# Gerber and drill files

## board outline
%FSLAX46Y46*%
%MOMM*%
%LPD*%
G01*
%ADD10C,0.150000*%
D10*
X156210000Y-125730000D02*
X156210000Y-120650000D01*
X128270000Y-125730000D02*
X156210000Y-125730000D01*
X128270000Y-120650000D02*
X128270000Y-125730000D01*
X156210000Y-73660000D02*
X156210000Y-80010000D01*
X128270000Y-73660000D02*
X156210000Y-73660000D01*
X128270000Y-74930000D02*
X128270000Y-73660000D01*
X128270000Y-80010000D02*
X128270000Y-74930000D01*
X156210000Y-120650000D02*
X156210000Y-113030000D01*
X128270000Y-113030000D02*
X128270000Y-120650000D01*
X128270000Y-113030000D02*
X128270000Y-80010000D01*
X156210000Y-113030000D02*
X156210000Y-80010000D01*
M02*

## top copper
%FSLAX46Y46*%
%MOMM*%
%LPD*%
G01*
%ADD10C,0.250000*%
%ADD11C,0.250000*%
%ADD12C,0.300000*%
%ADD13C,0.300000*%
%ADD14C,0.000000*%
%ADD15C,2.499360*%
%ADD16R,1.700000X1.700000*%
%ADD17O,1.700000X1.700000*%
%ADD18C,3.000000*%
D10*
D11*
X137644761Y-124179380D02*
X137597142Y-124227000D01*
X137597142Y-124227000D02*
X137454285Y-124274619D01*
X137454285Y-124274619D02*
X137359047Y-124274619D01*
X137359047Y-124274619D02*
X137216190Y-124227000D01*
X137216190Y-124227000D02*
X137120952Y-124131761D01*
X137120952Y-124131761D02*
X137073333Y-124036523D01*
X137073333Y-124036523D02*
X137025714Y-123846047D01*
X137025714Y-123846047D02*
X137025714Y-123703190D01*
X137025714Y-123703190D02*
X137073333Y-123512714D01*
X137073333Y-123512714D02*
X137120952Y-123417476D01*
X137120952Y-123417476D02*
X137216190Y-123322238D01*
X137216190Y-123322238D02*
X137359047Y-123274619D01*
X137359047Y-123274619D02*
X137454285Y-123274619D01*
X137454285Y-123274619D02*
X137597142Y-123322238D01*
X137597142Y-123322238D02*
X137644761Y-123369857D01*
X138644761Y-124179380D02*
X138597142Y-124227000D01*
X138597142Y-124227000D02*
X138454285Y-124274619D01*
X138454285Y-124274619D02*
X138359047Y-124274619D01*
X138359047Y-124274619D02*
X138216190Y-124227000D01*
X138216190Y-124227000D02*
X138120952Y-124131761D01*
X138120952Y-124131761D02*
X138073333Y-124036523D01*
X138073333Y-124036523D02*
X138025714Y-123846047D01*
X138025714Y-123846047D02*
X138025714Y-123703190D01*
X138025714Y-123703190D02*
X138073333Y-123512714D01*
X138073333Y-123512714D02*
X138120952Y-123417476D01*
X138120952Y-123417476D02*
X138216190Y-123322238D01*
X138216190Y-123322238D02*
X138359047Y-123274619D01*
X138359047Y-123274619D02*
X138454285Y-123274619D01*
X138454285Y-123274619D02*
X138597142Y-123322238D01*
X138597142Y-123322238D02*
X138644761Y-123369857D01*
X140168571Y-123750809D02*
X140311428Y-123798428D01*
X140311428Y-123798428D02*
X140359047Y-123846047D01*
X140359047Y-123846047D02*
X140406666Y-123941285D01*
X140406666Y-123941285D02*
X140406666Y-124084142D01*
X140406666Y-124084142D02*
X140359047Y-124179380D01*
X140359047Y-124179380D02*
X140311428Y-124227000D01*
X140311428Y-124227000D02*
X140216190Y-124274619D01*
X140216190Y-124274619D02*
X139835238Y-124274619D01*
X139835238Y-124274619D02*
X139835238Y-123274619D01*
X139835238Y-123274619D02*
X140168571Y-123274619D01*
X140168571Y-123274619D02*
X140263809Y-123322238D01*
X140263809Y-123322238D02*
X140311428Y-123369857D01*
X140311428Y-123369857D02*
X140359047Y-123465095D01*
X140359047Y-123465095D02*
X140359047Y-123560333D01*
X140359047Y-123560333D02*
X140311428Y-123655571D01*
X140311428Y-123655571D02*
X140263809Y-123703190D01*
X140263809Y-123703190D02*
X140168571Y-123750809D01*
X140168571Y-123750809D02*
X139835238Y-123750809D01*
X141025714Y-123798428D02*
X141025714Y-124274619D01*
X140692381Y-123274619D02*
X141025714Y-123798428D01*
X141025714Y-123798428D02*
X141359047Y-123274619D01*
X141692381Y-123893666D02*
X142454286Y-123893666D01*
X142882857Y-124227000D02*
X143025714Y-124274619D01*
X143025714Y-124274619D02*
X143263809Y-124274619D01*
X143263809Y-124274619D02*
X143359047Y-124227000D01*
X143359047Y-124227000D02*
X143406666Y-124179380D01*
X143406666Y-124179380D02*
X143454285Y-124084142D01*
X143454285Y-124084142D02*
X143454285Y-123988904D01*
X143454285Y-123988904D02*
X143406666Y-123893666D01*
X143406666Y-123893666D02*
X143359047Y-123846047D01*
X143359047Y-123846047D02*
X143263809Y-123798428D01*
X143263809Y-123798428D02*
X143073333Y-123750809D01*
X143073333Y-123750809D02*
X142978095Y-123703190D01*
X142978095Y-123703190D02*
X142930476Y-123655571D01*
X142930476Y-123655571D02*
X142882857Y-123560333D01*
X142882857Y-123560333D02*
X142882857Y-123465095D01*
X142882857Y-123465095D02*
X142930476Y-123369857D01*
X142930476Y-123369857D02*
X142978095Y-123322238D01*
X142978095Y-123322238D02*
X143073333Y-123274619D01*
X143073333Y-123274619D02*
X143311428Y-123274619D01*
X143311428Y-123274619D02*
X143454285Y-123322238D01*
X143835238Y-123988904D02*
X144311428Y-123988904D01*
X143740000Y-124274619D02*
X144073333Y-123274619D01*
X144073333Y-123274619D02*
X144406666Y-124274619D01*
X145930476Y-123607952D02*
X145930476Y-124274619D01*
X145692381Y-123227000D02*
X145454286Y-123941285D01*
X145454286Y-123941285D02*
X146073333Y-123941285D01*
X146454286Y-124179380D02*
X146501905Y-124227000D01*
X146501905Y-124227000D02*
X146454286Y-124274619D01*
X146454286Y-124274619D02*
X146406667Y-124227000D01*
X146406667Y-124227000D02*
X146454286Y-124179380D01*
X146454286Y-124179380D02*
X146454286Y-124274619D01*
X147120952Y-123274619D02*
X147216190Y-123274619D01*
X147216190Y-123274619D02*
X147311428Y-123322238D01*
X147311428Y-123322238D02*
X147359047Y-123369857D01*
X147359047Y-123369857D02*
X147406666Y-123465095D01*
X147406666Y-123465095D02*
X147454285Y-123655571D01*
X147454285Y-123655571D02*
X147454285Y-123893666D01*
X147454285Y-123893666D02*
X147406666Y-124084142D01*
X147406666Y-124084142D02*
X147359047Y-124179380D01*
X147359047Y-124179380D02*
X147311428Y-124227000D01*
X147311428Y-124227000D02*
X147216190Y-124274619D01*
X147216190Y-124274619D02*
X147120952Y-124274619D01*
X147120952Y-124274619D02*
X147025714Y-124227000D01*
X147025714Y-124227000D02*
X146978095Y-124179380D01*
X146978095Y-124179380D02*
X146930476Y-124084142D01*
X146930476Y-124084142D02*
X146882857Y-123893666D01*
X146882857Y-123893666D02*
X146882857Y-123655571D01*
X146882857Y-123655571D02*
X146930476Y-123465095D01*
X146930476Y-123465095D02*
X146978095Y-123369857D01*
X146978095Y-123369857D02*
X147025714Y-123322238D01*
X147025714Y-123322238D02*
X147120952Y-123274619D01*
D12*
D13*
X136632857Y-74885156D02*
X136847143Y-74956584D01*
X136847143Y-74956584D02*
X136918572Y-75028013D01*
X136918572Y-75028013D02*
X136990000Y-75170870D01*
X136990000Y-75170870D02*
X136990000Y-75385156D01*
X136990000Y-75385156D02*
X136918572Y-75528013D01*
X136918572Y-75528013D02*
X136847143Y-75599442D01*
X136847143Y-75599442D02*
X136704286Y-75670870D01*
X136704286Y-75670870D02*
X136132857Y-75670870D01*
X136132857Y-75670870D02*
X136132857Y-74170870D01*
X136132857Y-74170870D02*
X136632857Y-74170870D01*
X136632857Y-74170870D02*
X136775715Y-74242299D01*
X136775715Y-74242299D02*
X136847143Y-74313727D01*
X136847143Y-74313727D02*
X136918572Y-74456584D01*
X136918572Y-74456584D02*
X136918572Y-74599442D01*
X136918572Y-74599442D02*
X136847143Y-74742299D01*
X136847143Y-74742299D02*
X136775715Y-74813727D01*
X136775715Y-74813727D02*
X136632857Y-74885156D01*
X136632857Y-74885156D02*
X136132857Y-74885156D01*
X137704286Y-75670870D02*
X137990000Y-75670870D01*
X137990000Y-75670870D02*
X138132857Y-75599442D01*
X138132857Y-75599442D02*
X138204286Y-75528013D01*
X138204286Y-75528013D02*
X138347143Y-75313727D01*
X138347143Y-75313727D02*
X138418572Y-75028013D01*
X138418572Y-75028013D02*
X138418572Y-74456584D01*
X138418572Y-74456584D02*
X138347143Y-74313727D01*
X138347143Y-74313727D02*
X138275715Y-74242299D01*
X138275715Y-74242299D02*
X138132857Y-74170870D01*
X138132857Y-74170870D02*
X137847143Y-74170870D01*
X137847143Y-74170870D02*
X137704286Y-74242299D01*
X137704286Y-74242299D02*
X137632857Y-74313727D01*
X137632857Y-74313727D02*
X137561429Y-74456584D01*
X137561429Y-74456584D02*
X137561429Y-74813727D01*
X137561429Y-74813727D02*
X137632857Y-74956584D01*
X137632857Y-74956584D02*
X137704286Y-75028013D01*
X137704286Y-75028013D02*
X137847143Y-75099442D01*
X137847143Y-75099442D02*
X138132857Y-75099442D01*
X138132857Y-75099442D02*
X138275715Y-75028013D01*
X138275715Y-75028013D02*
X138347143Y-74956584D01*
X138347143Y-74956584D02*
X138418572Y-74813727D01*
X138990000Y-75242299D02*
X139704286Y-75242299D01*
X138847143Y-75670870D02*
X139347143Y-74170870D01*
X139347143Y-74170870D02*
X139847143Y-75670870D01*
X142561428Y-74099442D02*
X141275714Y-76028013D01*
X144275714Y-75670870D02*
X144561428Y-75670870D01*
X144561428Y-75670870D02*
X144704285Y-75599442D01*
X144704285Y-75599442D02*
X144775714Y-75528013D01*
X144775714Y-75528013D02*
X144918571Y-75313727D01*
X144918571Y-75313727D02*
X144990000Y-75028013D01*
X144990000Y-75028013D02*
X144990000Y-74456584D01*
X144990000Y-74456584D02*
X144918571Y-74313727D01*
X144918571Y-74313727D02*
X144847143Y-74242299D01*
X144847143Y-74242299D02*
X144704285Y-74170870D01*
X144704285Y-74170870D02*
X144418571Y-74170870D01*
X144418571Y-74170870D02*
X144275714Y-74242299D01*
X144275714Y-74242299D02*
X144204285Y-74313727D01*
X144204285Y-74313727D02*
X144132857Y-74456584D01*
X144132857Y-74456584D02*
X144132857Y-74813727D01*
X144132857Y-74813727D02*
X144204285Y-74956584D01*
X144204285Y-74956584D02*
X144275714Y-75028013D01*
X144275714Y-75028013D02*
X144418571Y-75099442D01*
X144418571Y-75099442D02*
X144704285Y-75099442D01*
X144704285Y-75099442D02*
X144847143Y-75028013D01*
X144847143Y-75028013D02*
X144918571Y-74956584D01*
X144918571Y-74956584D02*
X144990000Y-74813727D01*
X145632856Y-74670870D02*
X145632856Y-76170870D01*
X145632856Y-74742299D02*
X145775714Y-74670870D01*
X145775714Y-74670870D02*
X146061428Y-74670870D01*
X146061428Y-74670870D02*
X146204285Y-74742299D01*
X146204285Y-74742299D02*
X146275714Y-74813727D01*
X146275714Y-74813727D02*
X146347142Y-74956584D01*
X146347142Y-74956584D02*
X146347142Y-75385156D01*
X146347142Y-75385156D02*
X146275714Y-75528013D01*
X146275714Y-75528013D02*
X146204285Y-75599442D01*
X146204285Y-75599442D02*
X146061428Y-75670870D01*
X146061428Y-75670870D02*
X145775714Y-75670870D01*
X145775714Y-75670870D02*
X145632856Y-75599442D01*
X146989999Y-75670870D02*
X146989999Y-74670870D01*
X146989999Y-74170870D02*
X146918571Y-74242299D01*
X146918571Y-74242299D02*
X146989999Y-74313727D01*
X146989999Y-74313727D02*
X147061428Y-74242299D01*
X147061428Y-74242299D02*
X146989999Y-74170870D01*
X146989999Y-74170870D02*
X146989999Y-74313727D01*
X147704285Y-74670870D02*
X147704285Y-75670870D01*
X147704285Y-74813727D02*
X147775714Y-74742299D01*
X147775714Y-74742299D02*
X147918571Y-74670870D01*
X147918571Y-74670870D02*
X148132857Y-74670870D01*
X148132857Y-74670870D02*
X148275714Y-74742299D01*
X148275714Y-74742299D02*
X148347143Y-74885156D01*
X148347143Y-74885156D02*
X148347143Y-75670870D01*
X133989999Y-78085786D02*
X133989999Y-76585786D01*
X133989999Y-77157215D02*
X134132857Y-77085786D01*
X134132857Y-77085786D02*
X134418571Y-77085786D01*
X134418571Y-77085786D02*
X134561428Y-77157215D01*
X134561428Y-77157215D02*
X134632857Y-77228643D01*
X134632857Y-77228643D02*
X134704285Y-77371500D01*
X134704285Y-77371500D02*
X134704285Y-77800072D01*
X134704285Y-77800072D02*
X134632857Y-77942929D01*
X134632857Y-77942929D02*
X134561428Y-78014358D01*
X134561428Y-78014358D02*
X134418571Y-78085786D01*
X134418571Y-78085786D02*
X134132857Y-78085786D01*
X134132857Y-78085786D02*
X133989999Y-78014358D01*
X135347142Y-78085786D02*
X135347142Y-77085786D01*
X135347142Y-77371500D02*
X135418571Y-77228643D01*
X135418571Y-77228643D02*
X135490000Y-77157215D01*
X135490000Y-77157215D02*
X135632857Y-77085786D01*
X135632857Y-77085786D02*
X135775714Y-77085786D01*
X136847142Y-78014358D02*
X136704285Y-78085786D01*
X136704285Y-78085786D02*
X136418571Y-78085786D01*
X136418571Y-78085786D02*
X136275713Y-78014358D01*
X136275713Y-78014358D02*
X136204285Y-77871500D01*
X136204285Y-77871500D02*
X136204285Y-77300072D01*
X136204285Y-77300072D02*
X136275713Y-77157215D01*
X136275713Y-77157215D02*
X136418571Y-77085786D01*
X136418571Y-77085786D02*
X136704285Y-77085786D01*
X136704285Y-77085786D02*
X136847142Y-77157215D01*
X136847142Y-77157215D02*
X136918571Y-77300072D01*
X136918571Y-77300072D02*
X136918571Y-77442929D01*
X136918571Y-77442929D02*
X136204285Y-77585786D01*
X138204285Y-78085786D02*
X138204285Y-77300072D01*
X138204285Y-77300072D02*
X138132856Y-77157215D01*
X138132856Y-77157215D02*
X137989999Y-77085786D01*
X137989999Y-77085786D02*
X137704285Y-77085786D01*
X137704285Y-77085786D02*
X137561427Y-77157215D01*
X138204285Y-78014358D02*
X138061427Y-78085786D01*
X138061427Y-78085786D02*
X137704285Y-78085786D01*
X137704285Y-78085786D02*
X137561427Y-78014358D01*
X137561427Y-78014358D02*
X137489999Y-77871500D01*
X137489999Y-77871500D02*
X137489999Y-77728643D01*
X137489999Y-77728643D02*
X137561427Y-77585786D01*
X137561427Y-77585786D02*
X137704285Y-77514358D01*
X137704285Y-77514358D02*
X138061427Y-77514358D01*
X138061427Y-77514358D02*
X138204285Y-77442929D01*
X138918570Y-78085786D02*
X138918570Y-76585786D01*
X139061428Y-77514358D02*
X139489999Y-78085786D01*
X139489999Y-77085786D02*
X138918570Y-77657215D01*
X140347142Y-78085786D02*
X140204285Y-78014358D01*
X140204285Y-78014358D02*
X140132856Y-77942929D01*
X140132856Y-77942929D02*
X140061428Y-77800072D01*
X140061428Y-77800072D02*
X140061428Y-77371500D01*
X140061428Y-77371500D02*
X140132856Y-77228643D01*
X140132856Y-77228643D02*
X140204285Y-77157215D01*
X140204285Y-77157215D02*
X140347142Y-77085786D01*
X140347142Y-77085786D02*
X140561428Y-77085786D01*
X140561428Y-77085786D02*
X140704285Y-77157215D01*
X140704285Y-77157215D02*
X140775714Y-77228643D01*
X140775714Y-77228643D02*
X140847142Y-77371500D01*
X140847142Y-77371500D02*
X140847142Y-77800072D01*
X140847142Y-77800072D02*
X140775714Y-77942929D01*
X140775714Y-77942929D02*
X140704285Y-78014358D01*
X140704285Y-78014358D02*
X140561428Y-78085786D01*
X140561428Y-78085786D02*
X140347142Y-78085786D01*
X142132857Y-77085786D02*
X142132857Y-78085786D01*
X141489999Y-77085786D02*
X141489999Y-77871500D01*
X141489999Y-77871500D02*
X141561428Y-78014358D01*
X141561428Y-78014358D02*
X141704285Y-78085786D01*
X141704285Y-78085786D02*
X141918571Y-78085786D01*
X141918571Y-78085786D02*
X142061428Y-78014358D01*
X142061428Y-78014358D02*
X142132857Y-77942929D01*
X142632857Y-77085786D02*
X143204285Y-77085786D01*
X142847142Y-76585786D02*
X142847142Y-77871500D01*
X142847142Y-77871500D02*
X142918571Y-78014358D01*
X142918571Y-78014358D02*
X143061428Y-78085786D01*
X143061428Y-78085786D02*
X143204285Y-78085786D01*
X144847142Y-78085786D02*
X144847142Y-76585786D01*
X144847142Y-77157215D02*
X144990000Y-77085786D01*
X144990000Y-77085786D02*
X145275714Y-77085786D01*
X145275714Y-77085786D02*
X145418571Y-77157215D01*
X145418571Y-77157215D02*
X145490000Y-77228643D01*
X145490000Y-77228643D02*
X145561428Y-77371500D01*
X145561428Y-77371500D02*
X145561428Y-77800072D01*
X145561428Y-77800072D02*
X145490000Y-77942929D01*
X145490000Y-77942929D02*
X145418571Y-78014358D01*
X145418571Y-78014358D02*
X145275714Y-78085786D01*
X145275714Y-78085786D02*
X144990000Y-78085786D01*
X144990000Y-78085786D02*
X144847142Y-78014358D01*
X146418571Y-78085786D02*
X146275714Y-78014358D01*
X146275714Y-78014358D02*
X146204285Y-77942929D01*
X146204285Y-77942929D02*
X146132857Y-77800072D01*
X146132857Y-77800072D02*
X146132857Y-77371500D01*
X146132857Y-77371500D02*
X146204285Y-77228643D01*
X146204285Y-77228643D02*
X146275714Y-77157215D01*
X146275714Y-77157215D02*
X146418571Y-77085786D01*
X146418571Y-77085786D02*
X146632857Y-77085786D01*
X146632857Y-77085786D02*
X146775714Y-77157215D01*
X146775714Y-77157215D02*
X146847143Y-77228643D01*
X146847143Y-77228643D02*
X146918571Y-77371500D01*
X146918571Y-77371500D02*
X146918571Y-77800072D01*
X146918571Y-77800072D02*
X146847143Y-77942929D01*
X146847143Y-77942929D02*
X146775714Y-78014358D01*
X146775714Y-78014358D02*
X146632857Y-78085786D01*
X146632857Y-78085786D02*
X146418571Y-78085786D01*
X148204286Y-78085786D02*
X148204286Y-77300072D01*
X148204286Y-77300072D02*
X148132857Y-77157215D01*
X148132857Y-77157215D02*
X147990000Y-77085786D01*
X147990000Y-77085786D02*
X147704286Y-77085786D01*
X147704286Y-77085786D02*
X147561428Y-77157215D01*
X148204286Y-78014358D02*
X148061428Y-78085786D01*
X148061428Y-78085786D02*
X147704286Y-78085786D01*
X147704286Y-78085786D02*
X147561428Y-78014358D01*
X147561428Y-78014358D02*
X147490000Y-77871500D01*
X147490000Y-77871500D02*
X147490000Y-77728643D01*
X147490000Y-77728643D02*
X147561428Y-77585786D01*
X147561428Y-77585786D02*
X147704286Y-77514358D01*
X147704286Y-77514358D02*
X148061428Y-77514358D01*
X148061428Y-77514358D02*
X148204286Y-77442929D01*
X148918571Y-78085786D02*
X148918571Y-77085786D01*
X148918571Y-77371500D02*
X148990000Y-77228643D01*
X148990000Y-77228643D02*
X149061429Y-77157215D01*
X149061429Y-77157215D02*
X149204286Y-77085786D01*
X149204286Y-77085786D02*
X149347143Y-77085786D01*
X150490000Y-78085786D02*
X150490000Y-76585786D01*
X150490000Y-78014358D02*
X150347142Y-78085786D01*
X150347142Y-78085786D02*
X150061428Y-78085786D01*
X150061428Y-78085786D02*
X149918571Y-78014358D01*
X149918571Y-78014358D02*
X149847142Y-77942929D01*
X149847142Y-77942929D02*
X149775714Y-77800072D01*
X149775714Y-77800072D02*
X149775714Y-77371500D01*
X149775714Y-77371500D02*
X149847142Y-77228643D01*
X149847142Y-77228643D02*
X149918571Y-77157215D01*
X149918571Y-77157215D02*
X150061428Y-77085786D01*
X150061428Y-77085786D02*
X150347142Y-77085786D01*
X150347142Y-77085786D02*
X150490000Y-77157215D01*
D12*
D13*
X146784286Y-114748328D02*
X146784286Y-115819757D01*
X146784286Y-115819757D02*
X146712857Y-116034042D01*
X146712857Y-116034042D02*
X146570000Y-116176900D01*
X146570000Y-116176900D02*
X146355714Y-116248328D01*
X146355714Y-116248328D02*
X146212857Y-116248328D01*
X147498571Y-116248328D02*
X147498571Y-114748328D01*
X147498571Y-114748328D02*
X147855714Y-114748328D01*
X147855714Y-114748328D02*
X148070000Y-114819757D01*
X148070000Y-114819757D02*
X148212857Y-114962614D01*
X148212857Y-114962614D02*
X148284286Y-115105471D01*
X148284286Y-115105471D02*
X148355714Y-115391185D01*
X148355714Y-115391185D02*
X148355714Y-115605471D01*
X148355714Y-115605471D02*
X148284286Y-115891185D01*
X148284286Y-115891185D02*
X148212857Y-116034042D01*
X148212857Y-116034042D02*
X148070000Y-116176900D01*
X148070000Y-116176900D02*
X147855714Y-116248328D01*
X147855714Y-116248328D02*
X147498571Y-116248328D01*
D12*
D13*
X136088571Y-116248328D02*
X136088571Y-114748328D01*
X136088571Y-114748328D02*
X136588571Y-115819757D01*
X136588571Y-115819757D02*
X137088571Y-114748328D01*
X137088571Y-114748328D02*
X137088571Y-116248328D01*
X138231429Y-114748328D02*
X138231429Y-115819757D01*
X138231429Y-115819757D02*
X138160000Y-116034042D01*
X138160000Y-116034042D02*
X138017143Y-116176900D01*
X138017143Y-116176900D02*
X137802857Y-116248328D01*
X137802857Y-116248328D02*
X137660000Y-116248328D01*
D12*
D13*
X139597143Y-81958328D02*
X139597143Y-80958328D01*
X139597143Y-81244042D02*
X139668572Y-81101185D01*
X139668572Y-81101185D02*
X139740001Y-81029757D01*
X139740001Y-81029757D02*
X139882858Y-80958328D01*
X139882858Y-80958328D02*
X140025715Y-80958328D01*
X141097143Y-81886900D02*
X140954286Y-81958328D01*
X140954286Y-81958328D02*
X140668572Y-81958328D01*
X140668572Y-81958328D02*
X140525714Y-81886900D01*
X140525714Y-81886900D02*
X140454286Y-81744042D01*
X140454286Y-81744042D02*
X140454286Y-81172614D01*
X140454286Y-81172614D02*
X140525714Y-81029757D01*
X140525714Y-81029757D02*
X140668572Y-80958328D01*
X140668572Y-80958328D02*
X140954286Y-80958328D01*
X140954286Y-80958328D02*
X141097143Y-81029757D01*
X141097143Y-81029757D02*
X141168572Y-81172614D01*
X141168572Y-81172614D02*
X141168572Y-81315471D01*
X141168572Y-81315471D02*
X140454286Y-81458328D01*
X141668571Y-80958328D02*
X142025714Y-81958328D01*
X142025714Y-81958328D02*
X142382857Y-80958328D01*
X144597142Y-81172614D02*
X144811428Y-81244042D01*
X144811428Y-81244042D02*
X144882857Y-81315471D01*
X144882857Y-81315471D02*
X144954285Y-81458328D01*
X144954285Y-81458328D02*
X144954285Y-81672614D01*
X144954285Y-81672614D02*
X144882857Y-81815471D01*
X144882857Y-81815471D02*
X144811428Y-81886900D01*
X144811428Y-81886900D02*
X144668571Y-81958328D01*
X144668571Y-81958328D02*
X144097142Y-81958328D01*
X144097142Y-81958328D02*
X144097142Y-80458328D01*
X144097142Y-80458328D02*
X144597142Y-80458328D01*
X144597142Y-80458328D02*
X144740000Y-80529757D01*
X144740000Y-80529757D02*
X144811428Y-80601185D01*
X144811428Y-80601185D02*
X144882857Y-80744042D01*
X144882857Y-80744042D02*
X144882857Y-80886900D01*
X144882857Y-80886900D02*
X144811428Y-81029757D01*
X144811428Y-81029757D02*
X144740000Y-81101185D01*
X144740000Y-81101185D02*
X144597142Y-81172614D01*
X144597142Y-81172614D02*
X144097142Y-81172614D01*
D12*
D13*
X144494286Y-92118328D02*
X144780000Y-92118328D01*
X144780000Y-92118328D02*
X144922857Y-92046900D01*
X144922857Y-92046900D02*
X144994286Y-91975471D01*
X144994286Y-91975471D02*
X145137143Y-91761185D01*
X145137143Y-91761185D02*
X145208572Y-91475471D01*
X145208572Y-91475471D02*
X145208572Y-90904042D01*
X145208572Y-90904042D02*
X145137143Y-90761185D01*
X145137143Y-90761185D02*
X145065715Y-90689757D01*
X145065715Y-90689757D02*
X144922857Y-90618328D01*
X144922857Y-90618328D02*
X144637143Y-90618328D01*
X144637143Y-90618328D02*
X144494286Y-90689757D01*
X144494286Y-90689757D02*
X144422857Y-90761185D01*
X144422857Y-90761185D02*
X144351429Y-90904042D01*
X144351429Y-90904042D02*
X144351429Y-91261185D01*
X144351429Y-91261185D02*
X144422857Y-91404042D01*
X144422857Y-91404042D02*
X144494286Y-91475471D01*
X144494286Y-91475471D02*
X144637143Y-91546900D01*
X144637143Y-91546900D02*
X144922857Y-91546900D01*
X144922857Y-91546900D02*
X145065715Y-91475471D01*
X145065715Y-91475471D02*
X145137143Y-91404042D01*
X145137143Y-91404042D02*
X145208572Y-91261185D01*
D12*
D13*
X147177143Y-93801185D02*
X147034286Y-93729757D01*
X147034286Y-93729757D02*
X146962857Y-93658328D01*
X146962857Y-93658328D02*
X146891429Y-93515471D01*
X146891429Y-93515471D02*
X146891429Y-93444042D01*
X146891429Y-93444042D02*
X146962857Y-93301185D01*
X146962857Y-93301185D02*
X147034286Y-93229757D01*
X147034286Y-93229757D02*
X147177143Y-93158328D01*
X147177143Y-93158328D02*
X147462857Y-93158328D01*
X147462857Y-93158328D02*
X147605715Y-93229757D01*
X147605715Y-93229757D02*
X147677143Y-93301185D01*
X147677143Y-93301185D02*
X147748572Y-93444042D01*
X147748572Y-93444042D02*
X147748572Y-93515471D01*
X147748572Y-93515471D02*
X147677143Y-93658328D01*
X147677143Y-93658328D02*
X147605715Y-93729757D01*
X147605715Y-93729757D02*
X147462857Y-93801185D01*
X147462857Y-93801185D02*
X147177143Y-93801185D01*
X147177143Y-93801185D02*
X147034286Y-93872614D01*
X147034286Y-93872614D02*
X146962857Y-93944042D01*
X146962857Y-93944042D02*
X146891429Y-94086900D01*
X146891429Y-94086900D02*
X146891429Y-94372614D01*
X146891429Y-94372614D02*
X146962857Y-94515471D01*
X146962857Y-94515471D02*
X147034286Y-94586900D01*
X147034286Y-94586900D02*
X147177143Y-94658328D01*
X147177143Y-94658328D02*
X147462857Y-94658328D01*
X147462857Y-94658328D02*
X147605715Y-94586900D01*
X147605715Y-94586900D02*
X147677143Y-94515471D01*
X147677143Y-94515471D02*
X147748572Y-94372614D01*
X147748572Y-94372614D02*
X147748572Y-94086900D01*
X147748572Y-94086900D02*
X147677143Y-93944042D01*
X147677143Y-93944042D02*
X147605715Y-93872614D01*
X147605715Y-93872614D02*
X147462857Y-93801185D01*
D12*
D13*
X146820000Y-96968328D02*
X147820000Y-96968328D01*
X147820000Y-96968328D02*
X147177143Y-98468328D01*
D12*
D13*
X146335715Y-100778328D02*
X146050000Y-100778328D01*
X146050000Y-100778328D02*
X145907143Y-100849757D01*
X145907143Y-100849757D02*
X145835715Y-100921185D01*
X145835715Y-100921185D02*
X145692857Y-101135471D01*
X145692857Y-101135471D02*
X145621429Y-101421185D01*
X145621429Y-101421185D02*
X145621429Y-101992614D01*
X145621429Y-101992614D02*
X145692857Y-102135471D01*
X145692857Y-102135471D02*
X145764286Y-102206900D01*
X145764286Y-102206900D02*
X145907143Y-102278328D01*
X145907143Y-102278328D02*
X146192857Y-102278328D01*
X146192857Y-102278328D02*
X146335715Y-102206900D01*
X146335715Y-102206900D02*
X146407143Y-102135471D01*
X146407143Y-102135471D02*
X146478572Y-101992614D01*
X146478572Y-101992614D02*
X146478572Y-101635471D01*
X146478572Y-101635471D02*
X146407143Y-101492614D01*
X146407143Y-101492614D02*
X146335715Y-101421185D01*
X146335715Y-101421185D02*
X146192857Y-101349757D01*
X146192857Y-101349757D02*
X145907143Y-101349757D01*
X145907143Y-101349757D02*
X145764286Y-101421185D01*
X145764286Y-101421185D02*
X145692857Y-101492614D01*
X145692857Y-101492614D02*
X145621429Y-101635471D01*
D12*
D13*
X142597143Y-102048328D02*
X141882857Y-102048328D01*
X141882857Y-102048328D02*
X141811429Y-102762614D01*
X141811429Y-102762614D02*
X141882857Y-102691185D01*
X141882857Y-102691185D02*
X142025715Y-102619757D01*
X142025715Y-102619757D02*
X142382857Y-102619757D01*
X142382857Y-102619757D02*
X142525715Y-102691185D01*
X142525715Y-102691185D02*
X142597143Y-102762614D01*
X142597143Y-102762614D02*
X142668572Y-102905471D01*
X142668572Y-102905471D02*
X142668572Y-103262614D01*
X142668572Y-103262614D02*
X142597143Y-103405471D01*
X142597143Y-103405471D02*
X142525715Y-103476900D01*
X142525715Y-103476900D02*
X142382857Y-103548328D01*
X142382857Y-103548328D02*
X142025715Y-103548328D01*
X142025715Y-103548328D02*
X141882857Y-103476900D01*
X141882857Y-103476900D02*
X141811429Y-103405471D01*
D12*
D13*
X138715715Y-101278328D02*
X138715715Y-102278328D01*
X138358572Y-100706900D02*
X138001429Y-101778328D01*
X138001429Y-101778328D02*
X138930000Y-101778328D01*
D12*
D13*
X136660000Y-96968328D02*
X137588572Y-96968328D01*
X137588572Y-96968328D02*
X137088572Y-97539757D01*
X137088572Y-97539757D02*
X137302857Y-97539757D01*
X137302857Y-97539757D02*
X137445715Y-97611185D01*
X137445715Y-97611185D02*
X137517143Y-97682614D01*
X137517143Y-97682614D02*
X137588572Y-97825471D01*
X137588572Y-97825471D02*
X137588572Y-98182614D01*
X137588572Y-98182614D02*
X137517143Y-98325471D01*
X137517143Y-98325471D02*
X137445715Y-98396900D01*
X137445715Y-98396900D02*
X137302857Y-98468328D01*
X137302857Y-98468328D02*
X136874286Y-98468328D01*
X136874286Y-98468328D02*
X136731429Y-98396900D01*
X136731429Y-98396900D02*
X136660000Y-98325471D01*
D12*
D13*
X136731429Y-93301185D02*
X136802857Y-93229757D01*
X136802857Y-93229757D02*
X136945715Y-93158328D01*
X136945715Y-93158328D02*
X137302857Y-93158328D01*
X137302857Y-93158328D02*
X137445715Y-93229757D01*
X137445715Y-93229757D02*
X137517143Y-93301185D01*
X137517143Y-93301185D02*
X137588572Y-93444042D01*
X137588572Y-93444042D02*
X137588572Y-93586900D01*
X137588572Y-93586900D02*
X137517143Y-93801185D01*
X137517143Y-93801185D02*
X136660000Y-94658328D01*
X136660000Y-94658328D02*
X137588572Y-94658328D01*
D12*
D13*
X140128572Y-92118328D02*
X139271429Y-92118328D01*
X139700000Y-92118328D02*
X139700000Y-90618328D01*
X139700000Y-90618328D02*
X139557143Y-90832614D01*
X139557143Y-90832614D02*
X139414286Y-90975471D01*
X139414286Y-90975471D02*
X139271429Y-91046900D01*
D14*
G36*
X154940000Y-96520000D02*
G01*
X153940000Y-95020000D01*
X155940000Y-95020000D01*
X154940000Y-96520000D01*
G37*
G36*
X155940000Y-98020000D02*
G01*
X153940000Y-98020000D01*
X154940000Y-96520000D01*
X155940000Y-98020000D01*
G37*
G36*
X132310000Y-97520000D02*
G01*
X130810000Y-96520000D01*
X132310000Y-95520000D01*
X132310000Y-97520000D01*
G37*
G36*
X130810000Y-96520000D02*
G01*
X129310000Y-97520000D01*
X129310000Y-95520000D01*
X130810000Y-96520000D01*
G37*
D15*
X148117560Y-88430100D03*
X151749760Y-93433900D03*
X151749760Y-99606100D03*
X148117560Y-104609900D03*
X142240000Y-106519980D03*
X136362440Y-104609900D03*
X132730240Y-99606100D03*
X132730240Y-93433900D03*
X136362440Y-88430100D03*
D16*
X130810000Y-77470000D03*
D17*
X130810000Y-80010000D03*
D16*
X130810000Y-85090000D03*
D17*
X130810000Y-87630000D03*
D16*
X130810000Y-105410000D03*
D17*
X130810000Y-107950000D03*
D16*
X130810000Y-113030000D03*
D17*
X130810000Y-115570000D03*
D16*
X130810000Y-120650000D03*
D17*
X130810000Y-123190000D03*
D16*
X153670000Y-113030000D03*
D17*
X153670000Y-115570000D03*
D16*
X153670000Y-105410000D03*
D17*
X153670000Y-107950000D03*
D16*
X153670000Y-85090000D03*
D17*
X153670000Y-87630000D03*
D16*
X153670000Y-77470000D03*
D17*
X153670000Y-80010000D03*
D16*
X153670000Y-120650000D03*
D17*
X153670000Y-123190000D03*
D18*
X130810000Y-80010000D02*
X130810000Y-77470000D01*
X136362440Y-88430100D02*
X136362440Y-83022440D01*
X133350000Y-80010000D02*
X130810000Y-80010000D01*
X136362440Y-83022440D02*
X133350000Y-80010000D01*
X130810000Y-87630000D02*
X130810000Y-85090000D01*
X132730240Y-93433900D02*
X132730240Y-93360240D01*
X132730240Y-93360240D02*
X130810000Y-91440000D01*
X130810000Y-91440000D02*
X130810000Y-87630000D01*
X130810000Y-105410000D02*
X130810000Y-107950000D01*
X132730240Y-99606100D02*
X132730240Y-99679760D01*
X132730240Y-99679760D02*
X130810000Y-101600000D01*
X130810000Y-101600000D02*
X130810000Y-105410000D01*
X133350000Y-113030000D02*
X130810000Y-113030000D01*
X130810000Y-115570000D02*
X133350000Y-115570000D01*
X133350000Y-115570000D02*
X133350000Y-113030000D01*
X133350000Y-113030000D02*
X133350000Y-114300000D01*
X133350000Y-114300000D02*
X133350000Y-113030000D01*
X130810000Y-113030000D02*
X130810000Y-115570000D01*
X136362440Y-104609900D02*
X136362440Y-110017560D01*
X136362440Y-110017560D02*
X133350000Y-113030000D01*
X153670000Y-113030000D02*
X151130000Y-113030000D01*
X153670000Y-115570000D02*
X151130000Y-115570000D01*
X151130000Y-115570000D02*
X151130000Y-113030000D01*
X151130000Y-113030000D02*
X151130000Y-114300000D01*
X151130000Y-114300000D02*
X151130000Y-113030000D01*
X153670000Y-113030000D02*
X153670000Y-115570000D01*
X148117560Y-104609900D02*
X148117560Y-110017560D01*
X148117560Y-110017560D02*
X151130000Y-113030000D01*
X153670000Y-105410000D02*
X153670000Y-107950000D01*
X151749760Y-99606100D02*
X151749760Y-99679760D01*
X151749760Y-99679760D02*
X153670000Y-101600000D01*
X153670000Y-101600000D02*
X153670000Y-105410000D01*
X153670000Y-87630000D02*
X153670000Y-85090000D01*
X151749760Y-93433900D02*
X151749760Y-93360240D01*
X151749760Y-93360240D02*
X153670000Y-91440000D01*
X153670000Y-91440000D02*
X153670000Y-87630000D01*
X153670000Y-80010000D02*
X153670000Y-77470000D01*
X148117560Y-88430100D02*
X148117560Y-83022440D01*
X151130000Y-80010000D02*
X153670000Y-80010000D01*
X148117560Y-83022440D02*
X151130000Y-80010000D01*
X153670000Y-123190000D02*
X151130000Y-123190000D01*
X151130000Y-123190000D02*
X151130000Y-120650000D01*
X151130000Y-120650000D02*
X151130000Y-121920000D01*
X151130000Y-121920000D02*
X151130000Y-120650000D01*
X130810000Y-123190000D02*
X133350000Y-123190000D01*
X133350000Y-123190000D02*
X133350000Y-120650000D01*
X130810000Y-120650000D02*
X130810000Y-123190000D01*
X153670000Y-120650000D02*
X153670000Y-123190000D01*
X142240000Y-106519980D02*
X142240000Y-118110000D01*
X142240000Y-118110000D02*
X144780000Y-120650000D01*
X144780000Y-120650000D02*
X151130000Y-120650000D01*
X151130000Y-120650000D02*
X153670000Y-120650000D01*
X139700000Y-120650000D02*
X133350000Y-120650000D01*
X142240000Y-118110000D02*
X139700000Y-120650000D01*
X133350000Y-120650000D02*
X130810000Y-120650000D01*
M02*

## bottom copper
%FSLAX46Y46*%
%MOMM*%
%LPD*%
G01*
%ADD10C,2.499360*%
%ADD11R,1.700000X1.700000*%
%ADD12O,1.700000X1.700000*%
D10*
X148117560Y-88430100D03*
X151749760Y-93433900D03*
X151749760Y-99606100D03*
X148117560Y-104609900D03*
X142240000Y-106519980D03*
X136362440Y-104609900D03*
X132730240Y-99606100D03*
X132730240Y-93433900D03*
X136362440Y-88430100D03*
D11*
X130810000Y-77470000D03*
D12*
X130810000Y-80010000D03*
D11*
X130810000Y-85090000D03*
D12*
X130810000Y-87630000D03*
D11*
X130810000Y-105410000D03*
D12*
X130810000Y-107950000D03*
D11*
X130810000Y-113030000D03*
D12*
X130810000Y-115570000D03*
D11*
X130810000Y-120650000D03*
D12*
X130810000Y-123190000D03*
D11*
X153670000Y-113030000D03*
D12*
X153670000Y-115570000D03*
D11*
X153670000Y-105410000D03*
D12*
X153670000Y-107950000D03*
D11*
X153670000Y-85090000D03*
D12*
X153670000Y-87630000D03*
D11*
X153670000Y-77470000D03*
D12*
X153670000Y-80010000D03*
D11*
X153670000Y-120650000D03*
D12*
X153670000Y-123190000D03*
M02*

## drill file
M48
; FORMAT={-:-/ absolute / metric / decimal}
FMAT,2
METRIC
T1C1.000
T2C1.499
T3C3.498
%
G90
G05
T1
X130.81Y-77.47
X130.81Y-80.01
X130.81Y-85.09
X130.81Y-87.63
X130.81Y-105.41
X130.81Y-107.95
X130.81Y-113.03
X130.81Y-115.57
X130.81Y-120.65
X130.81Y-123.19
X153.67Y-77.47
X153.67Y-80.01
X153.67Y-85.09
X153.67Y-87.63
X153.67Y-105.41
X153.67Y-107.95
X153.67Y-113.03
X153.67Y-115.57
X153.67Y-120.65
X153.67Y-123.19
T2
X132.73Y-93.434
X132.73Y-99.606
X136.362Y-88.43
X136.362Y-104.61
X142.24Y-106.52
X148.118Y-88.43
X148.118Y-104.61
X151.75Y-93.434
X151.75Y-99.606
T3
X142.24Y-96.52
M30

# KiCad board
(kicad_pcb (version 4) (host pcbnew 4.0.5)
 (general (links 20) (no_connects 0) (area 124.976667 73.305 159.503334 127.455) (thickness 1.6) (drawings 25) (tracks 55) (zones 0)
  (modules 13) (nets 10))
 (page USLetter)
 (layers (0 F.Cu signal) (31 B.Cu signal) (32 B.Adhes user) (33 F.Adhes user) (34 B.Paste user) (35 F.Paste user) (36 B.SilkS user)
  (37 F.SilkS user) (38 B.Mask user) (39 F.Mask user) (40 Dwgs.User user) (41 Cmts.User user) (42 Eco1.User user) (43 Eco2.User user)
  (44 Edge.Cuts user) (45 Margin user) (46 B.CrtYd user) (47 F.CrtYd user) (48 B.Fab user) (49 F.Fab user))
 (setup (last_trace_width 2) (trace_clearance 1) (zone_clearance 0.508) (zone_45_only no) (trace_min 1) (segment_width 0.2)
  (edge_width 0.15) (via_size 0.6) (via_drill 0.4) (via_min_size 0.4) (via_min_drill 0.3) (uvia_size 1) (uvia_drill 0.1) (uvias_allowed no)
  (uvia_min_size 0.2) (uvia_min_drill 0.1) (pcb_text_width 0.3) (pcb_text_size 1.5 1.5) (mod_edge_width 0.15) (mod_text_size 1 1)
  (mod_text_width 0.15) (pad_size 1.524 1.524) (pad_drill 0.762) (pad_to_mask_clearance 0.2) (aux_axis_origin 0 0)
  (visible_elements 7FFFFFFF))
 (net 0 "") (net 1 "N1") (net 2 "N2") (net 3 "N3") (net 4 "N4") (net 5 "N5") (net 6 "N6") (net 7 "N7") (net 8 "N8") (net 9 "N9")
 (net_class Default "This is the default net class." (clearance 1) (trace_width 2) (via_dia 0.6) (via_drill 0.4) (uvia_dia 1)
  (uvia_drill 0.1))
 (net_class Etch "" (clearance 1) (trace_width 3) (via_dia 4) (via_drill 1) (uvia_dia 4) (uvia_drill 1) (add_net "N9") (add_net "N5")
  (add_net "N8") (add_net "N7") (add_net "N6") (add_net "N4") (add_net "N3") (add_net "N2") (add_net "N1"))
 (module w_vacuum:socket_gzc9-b (layer F.Cu) (at 142.24 96.52 180)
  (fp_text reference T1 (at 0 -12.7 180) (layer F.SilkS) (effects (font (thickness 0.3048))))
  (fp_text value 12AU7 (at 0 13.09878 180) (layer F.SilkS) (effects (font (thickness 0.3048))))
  (pad 9 thru_hole circle (at -5.87756 8.0899 180) (size 2.49936 2.49936) (drill 1.4986) (layers *.Cu *.Mask F.SilkS) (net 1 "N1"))
  (pad 8 thru_hole circle (at -9.50976 3.0861 180) (size 2.49936 2.49936) (drill 1.4986) (layers *.Cu *.Mask F.SilkS) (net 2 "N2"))
  (pad 7 thru_hole circle (at -9.50976 -3.0861 180) (size 2.49936 2.49936) (drill 1.4986) (layers *.Cu *.Mask F.SilkS) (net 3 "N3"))
  (pad 6 thru_hole circle (at -5.87756 -8.0899 180) (size 2.49936 2.49936) (drill 1.4986) (layers *.Cu *.Mask F.SilkS) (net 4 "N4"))
  (pad 5 thru_hole circle (at 0 -9.99998 180) (size 2.49936 2.49936) (drill 1.4986) (layers *.Cu *.Mask F.SilkS) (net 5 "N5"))
  (pad 4 thru_hole circle (at 5.87756 -8.0899 180) (size 2.49936 2.49936) (drill 1.4986) (layers *.Cu *.Mask F.SilkS) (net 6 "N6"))
  (pad 3 thru_hole circle (at 9.50976 -3.0861 180) (size 2.49936 2.49936) (drill 1.4986) (layers *.Cu *.Mask F.SilkS) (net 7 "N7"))
  (pad 2 thru_hole circle (at 9.50976 3.0861 180) (size 2.49936 2.49936) (drill 1.4986) (layers *.Cu *.Mask F.SilkS) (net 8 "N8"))
  (pad 1 thru_hole circle (at 5.87756 8.0899 180) (size 2.49936 2.49936) (drill 1.4986) (layers *.Cu *.Mask F.SilkS) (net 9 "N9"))
  (pad "" np_thru_hole circle (at 0 0 180) (size 3.49758 3.49758) (drill 3.49758) (layers *.Cu *.Mask F.SilkS)))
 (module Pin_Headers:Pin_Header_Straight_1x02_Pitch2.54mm (layer F.Cu) (at 130.81 77.47)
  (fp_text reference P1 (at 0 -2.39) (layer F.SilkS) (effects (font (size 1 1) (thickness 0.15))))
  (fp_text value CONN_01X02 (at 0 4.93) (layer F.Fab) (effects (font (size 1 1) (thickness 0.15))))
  (pad 1 thru_hole rect (at 0 0) (size 1.7 1.7) (drill 1) (layers *.Cu *.Mask) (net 9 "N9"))
  (pad 2 thru_hole oval (at 0 2.54) (size 1.7 1.7) (drill 1) (layers *.Cu *.Mask) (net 9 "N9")))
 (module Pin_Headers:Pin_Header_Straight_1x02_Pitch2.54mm (layer F.Cu) (at 130.81 85.09)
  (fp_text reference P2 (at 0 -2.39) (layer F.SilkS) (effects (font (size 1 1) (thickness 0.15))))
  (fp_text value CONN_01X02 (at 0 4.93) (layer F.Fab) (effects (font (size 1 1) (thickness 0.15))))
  (pad 1 thru_hole rect (at 0 0) (size 1.7 1.7) (drill 1) (layers *.Cu *.Mask) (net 8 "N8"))
  (pad 2 thru_hole oval (at 0 2.54) (size 1.7 1.7) (drill 1) (layers *.Cu *.Mask) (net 8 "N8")))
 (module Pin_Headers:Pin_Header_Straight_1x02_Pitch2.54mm (layer F.Cu) (at 130.81 105.41)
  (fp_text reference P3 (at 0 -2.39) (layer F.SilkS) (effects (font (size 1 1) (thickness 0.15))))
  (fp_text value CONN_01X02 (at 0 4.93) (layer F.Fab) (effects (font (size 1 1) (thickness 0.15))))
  (pad 1 thru_hole rect (at 0 0) (size 1.7 1.7) (drill 1) (layers *.Cu *.Mask) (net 7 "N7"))
  (pad 2 thru_hole oval (at 0 2.54) (size 1.7 1.7) (drill 1) (layers *.Cu *.Mask) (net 7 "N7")))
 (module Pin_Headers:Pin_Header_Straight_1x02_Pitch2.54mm (layer F.Cu) (at 130.81 113.03)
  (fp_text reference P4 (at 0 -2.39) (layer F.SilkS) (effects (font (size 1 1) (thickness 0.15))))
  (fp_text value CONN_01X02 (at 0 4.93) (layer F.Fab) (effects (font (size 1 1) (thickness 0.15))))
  (pad 1 thru_hole rect (at 0 0) (size 1.7 1.7) (drill 1) (layers *.Cu *.Mask) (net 6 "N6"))
  (pad 2 thru_hole oval (at 0 2.54) (size 1.7 1.7) (drill 1) (layers *.Cu *.Mask) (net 6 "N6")))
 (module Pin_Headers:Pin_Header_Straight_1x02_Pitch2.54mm (layer F.Cu) (at 130.81 120.65)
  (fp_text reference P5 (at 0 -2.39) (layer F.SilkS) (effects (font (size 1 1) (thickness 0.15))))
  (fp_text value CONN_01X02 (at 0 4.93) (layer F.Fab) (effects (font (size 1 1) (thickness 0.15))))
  (pad 1 thru_hole rect (at 0 0) (size 1.7 1.7) (drill 1) (layers *.Cu *.Mask) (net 5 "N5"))
  (pad 2 thru_hole oval (at 0 2.54) (size 1.7 1.7) (drill 1) (layers *.Cu *.Mask) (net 5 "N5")))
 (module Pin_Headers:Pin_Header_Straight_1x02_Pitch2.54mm (layer F.Cu) (at 153.67 113.03)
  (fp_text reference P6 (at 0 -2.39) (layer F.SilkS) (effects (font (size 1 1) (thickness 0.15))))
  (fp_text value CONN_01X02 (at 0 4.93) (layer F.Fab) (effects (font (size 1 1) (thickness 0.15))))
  (pad 1 thru_hole rect (at 0 0) (size 1.7 1.7) (drill 1) (layers *.Cu *.Mask) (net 4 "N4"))
  (pad 2 thru_hole oval (at 0 2.54) (size 1.7 1.7) (drill 1) (layers *.Cu *.Mask) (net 4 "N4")))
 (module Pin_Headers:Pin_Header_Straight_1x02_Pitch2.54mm (layer F.Cu) (at 153.67 105.41)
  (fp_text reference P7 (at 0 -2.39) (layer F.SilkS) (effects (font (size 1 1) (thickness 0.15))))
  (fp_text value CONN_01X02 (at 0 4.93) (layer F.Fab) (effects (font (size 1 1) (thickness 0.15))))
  (pad 1 thru_hole rect (at 0 0) (size 1.7 1.7) (drill 1) (layers *.Cu *.Mask) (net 3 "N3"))
  (pad 2 thru_hole oval (at 0 2.54) (size 1.7 1.7) (drill 1) (layers *.Cu *.Mask) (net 3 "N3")))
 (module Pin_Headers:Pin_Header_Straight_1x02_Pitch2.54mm (layer F.Cu) (at 153.67 85.09)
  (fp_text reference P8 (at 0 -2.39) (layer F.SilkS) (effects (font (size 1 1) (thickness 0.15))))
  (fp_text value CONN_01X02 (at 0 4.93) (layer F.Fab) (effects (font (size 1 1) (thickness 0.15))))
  (pad 1 thru_hole rect (at 0 0) (size 1.7 1.7) (drill 1) (layers *.Cu *.Mask) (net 2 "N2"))
  (pad 2 thru_hole oval (at 0 2.54) (size 1.7 1.7) (drill 1) (layers *.Cu *.Mask) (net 2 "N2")))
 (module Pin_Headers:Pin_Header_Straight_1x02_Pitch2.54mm (layer F.Cu) (at 153.67 77.47)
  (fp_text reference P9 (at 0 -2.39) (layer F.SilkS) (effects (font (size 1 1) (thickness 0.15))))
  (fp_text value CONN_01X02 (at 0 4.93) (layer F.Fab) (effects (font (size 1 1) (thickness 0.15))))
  (pad 1 thru_hole rect (at 0 0) (size 1.7 1.7) (drill 1) (layers *.Cu *.Mask) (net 1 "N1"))
  (pad 2 thru_hole oval (at 0 2.54) (size 1.7 1.7) (drill 1) (layers *.Cu *.Mask) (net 1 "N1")))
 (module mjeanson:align (layer F.Cu) (at 154.94 96.52 90)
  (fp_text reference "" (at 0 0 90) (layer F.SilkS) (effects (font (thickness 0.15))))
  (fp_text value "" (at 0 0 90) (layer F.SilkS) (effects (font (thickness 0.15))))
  (fp_poly (pts (xy 0 0) (xy 1.5 -1) (xy 1.5 1) (xy 0 0)) (layer F.Cu) (width 0))
  (fp_poly (pts (xy 0 0) (xy -1.5 1) (xy -1.5 -1) (xy 0 0)) (layer F.Cu) (width 0)))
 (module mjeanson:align (layer F.Cu) (at 130.81 96.52)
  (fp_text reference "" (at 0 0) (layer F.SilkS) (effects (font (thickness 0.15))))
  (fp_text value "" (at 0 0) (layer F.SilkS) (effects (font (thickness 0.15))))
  (fp_poly (pts (xy 0 0) (xy 1.5 -1) (xy 1.5 1) (xy 0 0)) (layer F.Cu) (width 0))
  (fp_poly (pts (xy 0 0) (xy -1.5 1) (xy -1.5 -1) (xy 0 0)) (layer F.Cu) (width 0)))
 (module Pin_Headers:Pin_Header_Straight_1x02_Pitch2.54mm (layer F.Cu) (at 153.67 120.65)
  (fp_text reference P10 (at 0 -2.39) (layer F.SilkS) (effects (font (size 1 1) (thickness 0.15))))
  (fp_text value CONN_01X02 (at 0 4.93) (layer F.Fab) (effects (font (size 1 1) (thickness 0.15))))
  (pad 1 thru_hole rect (at 0 0) (size 1.7 1.7) (drill 1) (layers *.Cu *.Mask) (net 5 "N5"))
  (pad 2 thru_hole oval (at 0 2.54) (size 1.7 1.7) (drill 1) (layers *.Cu *.Mask) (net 5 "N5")))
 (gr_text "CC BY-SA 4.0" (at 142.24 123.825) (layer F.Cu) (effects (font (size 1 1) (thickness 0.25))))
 (gr_line (start 156.21 125.73) (end 156.21 120.65) (angle 90) (layer Edge.Cuts) (width 0.15))
 (gr_line (start 128.27 125.73) (end 156.21 125.73) (angle 90) (layer Edge.Cuts) (width 0.15))
 (gr_line (start 128.27 120.65) (end 128.27 125.73) (angle 90) (layer Edge.Cuts) (width 0.15))
 (gr_line (start 156.21 73.66) (end 156.21 80.01) (angle 90) (layer Edge.Cuts) (width 0.15))
 (gr_line (start 128.27 73.66) (end 156.21 73.66) (angle 90) (layer Edge.Cuts) (width 0.15))
 (gr_line (start 128.27 74.93) (end 128.27 73.66) (angle 90) (layer Edge.Cuts) (width 0.15))
 (gr_line (start 128.27 80.01) (end 128.27 74.93) (angle 90) (layer Edge.Cuts) (width 0.15))
 (gr_line (start 156.21 120.65) (end 156.21 113.03) (angle 90) (layer Edge.Cuts) (width 0.15))
 (gr_line (start 128.27 113.03) (end 128.27 120.65) (angle 90) (layer Edge.Cuts) (width 0.15))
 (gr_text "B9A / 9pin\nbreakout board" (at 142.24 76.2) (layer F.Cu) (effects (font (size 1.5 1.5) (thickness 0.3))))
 (gr_line (start 128.27 113.03) (end 128.27 80.01) (angle 90) (layer Edge.Cuts) (width 0.15))
 (gr_line (start 156.21 113.03) (end 156.21 80.01) (angle 90) (layer Edge.Cuts) (width 0.15))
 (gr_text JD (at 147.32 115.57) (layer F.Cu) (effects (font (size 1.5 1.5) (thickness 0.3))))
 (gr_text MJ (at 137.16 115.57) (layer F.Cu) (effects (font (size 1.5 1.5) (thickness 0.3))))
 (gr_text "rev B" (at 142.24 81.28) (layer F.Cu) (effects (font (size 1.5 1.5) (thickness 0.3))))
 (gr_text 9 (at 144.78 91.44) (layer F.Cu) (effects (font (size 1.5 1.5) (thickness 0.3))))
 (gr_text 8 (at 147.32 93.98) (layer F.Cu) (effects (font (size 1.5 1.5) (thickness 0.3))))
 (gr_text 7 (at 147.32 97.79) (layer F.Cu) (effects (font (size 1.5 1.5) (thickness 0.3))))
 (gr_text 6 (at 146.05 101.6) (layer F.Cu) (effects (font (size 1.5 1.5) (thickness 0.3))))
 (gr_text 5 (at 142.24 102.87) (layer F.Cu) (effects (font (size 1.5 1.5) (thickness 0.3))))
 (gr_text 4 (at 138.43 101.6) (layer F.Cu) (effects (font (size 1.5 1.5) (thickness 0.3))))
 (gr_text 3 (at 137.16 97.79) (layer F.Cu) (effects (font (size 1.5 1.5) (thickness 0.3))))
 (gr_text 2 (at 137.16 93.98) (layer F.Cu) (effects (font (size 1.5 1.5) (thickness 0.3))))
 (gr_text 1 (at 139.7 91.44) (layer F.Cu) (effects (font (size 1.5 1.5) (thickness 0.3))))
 (segment (start 130.81 80.01) (end 130.81 77.47) (width 3) (layer F.Cu) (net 9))
 (segment (start 136.36244 88.4301) (end 136.36244 83.02244) (width 3) (layer F.Cu) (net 9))
 (segment (start 133.35 80.01) (end 130.81 80.01) (width 3) (layer F.Cu) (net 9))
 (segment (start 136.36244 83.02244) (end 133.35 80.01) (width 3) (layer F.Cu) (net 9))
 (segment (start 130.81 87.63) (end 130.81 85.09) (width 3) (layer F.Cu) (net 8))
 (segment (start 132.73024 93.4339) (end 132.73024 93.36024) (width 3) (layer F.Cu) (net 8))
 (segment (start 132.73024 93.36024) (end 130.81 91.44) (width 3) (layer F.Cu) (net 8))
 (segment (start 130.81 91.44) (end 130.81 87.63) (width 3) (layer F.Cu) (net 8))
 (segment (start 130.81 105.41) (end 130.81 107.95) (width 3) (layer F.Cu) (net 7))
 (segment (start 132.73024 99.6061) (end 132.73024 99.67976) (width 3) (layer F.Cu) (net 7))
 (segment (start 132.73024 99.67976) (end 130.81 101.6) (width 3) (layer F.Cu) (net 7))
 (segment (start 130.81 101.6) (end 130.81 105.41) (width 3) (layer F.Cu) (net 7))
 (segment (start 133.35 113.03) (end 130.81 113.03) (width 3) (layer F.Cu) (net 6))
 (segment (start 130.81 115.57) (end 133.35 115.57) (width 3) (layer F.Cu) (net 6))
 (segment (start 133.35 115.57) (end 133.35 113.03) (width 3) (layer F.Cu) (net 6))
 (segment (start 133.35 113.03) (end 133.35 114.3) (width 3) (layer F.Cu) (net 6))
 (segment (start 133.35 114.3) (end 133.35 113.03) (width 3) (layer F.Cu) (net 6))
 (segment (start 130.81 113.03) (end 130.81 115.57) (width 3) (layer F.Cu) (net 6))
 (segment (start 136.36244 104.6099) (end 136.36244 110.01756) (width 3) (layer F.Cu) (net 6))
 (segment (start 136.36244 110.01756) (end 133.35 113.03) (width 3) (layer F.Cu) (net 6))
 (segment (start 153.67 113.03) (end 151.13 113.03) (width 3) (layer F.Cu) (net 4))
 (segment (start 153.67 115.57) (end 151.13 115.57) (width 3) (layer F.Cu) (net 4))
 (segment (start 151.13 115.57) (end 151.13 113.03) (width 3) (layer F.Cu) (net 4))
 (segment (start 151.13 113.03) (end 151.13 114.3) (width 3) (layer F.Cu) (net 4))
 (segment (start 151.13 114.3) (end 151.13 113.03) (width 3) (layer F.Cu) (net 4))
 (segment (start 153.67 113.03) (end 153.67 115.57) (width 3) (layer F.Cu) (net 4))
 (segment (start 148.11756 104.6099) (end 148.11756 110.01756) (width 3) (layer F.Cu) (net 4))
 (segment (start 148.11756 110.01756) (end 151.13 113.03) (width 3) (layer F.Cu) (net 4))
 (segment (start 153.67 105.41) (end 153.67 107.95) (width 3) (layer F.Cu) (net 3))
 (segment (start 151.74976 99.6061) (end 151.74976 99.67976) (width 3) (layer F.Cu) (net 3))
 (segment (start 151.74976 99.67976) (end 153.67 101.6) (width 3) (layer F.Cu) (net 3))
 (segment (start 153.67 101.6) (end 153.67 105.41) (width 3) (layer F.Cu) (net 3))
 (segment (start 153.67 87.63) (end 153.67 85.09) (width 3) (layer F.Cu) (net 2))
 (segment (start 151.74976 93.4339) (end 151.74976 93.36024) (width 3) (layer F.Cu) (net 2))
 (segment (start 151.74976 93.36024) (end 153.67 91.44) (width 3) (layer F.Cu) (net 2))
 (segment (start 153.67 91.44) (end 153.67 87.63) (width 3) (layer F.Cu) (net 2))
 (segment (start 153.67 80.01) (end 153.67 77.47) (width 3) (layer F.Cu) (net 1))
 (segment (start 148.11756 88.4301) (end 148.11756 83.02244) (width 3) (layer F.Cu) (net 1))
 (segment (start 151.13 80.01) (end 153.67 80.01) (width 3) (layer F.Cu) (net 1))
 (segment (start 148.11756 83.02244) (end 151.13 80.01) (width 3) (layer F.Cu) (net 1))
 (segment (start 153.67 123.19) (end 151.13 123.19) (width 3) (layer F.Cu) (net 5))
 (segment (start 151.13 123.19) (end 151.13 120.65) (width 3) (layer F.Cu) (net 5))
 (segment (start 151.13 120.65) (end 151.13 121.92) (width 3) (layer F.Cu) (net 5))
 (segment (start 151.13 121.92) (end 151.13 120.65) (width 3) (layer F.Cu) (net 5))
 (segment (start 130.81 123.19) (end 133.35 123.19) (width 3) (layer F.Cu) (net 5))
 (segment (start 133.35 123.19) (end 133.35 120.65) (width 3) (layer F.Cu) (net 5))
 (segment (start 130.81 120.65) (end 130.81 123.19) (width 3) (layer F.Cu) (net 5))
 (segment (start 153.67 120.65) (end 153.67 123.19) (width 3) (layer F.Cu) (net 5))
 (segment (start 142.24 106.51998) (end 142.24 118.11) (width 3) (layer F.Cu) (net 5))
 (segment (start 142.24 118.11) (end 144.78 120.65) (width 3) (layer F.Cu) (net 5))
 (segment (start 144.78 120.65) (end 151.13 120.65) (width 3) (layer F.Cu) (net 5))
 (segment (start 151.13 120.65) (end 153.67 120.65) (width 3) (layer F.Cu) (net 5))
 (segment (start 139.7 120.65) (end 133.35 120.65) (width 3) (layer F.Cu) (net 5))
 (segment (start 142.24 118.11) (end 139.7 120.65) (width 3) (layer F.Cu) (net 5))
 (segment (start 133.35 120.65) (end 130.81 120.65) (width 3) (layer F.Cu) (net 5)))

